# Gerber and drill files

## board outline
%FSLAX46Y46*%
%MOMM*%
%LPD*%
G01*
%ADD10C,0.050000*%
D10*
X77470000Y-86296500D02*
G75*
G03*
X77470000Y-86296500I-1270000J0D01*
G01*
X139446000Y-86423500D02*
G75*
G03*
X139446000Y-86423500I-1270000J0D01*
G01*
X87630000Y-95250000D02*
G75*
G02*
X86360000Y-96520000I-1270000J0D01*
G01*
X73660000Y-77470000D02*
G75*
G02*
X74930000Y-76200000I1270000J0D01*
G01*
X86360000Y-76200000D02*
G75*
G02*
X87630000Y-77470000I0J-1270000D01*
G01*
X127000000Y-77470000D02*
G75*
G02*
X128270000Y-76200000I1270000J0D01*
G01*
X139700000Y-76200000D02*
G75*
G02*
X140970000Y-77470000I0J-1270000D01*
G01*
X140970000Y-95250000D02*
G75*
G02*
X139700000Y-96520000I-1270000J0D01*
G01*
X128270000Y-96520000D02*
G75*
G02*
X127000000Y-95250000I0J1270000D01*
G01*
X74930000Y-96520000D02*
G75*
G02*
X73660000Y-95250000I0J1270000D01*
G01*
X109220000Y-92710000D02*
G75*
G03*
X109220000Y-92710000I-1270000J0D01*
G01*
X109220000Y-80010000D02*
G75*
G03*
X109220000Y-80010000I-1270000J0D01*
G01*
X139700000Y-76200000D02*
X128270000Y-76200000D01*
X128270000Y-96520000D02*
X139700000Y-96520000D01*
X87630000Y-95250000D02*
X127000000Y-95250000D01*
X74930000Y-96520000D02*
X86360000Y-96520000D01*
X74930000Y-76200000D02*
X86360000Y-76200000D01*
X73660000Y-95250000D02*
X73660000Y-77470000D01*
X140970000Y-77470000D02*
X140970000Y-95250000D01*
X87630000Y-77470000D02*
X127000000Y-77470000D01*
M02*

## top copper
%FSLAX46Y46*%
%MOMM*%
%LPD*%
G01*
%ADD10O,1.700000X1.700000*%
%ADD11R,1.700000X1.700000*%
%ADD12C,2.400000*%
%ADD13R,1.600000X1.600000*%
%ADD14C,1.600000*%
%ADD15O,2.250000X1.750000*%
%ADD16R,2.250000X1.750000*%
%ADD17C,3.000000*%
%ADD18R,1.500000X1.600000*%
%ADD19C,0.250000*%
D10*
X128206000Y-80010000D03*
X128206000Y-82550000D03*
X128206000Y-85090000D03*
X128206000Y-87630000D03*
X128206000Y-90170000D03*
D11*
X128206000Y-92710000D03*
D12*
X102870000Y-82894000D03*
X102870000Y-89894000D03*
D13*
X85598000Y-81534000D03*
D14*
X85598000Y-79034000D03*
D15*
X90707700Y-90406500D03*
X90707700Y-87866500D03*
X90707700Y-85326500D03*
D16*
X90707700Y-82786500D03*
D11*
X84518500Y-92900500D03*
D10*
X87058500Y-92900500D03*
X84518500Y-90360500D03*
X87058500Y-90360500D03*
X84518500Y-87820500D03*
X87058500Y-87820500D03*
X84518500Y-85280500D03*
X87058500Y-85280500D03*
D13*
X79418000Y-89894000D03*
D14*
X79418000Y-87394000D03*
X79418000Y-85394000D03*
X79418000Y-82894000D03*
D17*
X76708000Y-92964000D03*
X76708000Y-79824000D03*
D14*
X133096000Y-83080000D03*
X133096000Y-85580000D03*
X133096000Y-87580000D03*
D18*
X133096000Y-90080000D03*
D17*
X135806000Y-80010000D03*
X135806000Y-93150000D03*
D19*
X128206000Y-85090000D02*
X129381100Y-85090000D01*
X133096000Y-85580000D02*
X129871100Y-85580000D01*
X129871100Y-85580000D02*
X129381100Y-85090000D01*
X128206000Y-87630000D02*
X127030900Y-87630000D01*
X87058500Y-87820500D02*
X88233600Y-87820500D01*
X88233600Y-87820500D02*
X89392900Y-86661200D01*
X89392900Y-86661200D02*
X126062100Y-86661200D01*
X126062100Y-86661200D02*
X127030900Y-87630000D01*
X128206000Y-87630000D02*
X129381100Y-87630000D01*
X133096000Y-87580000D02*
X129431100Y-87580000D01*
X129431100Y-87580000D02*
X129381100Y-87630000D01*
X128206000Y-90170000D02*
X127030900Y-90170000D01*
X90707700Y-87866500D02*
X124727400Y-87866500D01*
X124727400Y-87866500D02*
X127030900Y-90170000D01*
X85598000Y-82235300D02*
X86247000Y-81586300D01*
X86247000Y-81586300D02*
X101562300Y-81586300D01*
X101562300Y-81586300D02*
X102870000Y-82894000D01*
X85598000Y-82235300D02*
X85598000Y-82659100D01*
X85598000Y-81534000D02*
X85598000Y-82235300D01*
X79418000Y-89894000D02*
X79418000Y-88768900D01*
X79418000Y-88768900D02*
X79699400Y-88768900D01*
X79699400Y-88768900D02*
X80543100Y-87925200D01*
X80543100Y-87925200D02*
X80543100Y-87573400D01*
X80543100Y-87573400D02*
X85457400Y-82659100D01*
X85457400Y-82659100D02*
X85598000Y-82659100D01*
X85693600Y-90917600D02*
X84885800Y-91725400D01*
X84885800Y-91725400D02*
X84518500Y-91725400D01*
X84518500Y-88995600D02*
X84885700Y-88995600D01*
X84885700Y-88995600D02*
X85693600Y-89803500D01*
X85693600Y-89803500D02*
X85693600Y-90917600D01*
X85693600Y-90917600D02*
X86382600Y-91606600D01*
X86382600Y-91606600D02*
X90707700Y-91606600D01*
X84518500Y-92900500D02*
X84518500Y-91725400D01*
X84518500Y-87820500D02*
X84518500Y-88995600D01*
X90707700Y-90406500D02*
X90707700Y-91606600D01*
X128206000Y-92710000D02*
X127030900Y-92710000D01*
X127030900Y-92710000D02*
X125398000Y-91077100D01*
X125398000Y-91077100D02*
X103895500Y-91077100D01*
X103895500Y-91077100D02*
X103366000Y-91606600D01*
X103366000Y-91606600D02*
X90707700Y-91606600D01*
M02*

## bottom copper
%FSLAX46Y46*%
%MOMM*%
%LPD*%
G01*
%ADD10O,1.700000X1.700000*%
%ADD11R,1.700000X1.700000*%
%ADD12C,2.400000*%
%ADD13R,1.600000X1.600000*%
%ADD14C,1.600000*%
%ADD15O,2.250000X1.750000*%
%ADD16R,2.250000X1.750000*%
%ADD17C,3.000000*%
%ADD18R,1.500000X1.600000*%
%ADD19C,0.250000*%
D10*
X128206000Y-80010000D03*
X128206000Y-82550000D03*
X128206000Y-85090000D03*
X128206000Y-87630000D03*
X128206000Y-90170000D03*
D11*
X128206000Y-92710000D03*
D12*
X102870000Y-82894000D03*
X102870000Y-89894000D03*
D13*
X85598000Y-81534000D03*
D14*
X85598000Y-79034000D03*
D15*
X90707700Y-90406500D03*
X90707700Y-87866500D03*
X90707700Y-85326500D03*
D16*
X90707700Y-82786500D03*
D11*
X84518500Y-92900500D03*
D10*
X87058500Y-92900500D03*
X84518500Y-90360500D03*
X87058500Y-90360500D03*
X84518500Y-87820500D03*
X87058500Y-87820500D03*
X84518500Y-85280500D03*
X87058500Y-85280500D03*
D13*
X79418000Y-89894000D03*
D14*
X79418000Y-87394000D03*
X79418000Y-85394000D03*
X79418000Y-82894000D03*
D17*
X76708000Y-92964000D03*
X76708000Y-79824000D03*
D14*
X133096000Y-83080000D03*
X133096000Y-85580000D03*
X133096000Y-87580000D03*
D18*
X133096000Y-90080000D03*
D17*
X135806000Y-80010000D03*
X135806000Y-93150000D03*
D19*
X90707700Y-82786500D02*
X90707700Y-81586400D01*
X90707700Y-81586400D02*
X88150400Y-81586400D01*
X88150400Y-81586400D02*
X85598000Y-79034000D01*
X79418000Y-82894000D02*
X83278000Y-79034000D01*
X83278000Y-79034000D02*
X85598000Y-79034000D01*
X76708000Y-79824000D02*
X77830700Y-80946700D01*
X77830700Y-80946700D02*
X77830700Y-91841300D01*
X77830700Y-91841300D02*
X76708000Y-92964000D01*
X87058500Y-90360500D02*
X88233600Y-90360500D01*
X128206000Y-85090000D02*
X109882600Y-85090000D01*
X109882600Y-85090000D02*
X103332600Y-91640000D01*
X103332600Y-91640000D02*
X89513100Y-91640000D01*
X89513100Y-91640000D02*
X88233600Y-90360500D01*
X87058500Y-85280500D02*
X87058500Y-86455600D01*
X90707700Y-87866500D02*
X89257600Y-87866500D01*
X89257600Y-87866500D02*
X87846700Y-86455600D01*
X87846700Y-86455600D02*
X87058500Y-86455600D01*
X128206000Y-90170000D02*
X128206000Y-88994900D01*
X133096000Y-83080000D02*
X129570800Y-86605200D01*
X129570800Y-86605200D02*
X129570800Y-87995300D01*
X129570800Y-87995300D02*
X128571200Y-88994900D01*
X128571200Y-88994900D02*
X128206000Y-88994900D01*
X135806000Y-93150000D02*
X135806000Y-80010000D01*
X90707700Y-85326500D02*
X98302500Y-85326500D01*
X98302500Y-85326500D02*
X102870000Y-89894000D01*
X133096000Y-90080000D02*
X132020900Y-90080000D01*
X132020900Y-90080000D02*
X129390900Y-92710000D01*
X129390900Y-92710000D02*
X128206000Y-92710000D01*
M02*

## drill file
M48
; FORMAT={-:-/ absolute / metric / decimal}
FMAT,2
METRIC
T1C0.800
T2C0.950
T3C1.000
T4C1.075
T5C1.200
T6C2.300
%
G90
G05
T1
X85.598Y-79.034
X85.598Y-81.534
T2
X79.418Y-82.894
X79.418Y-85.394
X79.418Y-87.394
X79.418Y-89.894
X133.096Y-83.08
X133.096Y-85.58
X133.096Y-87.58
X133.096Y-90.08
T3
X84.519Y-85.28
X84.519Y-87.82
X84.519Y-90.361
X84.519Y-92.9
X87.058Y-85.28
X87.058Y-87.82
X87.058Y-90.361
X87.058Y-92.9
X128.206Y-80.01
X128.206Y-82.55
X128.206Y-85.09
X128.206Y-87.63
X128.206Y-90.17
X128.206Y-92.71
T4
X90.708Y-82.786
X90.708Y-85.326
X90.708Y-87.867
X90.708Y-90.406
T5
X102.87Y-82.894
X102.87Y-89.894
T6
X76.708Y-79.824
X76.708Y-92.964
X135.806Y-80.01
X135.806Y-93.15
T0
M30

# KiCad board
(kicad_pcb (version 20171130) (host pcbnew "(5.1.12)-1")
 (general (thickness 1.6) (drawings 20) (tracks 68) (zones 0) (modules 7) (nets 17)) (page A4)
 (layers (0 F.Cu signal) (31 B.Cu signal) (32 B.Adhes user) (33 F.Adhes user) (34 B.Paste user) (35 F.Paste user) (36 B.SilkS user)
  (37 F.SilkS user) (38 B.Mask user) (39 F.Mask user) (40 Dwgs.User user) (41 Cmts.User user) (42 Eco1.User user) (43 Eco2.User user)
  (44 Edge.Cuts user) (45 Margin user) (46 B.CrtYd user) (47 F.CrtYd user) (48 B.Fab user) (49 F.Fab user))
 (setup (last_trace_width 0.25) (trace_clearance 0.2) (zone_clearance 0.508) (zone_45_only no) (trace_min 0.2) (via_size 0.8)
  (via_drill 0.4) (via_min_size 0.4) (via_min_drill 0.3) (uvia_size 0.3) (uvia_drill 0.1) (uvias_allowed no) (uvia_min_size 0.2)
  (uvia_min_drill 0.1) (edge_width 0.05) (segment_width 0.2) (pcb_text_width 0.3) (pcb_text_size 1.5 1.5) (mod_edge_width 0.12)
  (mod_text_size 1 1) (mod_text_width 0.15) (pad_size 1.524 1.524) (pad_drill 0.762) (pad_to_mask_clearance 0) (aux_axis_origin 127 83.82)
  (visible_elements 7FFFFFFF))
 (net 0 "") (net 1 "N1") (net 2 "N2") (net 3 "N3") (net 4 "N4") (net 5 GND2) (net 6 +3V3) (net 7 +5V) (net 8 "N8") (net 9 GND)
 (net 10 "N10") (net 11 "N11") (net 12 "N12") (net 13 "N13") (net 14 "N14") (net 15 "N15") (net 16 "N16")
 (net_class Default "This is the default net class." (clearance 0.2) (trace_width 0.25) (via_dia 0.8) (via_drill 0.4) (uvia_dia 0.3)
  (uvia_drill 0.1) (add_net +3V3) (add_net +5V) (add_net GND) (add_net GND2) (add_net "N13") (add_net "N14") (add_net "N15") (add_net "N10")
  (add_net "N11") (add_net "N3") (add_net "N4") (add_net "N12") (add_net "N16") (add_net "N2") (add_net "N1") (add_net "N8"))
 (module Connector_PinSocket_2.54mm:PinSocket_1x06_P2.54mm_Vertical (layer F.Cu) (at 128.206 92.71 180)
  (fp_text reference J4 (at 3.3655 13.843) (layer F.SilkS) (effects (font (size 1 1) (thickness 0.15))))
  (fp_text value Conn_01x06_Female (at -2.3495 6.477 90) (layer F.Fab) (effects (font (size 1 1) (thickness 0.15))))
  (pad 6 thru_hole oval (at 0 12.7 180) (size 1.7 1.7) (drill 1) (layers *.Cu *.Mask) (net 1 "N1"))
  (pad 5 thru_hole oval (at 0 10.16 180) (size 1.7 1.7) (drill 1) (layers *.Cu *.Mask) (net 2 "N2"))
  (pad 4 thru_hole oval (at 0 7.62 180) (size 1.7 1.7) (drill 1) (layers *.Cu *.Mask) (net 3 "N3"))
  (pad 3 thru_hole oval (at 0 5.08 180) (size 1.7 1.7) (drill 1) (layers *.Cu *.Mask) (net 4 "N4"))
  (pad 2 thru_hole oval (at 0 2.54 180) (size 1.7 1.7) (drill 1) (layers *.Cu *.Mask) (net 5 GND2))
  (pad 1 thru_hole rect (at 0 0 180) (size 1.7 1.7) (drill 1) (layers *.Cu *.Mask) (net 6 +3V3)))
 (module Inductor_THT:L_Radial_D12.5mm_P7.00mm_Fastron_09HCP (layer F.Cu) (at 102.87 82.894 270)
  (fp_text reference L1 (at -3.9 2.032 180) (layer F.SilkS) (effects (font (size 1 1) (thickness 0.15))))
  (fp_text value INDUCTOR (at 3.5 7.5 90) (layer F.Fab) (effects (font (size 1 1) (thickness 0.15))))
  (pad 1 thru_hole circle (at 0 0 270) (size 2.4 2.4) (drill 1.2) (layers *.Cu *.Mask) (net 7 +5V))
  (pad 2 thru_hole circle (at 7 0 270) (size 2.4 2.4) (drill 1.2) (layers *.Cu *.Mask) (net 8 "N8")))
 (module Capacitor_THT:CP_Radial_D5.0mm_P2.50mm (layer F.Cu) (at 85.598 81.534 90)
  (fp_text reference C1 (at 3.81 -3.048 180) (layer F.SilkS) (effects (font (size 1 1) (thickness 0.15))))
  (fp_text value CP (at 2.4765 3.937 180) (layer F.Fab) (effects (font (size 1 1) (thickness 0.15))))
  (pad 1 thru_hole rect (at 0 0 90) (size 1.6 1.6) (drill 0.8) (layers *.Cu *.Mask) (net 7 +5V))
  (pad 2 thru_hole circle (at 2.5 0 90) (size 1.6 1.6) (drill 0.8) (layers *.Cu *.Mask) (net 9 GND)))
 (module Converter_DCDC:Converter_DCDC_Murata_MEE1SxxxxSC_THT (layer F.Cu) (at 90.7077 82.7865)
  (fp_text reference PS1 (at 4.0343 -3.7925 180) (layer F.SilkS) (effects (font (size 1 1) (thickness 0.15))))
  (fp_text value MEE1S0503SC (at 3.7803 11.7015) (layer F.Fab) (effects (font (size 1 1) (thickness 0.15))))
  (pad 4 thru_hole oval (at 0 7.62 270) (size 1.75 2.25) (drill 1.075) (layers *.Cu *.Mask) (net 6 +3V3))
  (pad 3 thru_hole oval (at 0 5.08 270) (size 1.75 2.25) (drill 1.075) (layers *.Cu *.Mask) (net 5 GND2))
  (pad 2 thru_hole oval (at 0 2.54 270) (size 1.75 2.25) (drill 1.075) (layers *.Cu *.Mask) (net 8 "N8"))
  (pad 1 thru_hole rect (at 0 0 270) (size 1.75 2.25) (drill 1.075) (layers *.Cu *.Mask) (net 9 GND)))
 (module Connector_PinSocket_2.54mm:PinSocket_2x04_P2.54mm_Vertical (layer F.Cu) (at 84.5185 92.9005 180)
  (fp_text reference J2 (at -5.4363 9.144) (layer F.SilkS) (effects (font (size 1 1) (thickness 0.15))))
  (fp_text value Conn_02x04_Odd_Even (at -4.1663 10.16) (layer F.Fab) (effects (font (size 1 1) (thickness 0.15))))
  (pad 1 thru_hole rect (at 0 0 180) (size 1.7 1.7) (drill 1) (layers *.Cu *.Mask) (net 6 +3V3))
  (pad 2 thru_hole oval (at -2.54 0 180) (size 1.7 1.7) (drill 1) (layers *.Cu *.Mask) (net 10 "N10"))
  (pad 3 thru_hole oval (at 0 2.54 180) (size 1.7 1.7) (drill 1) (layers *.Cu *.Mask) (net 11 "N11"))
  (pad 4 thru_hole oval (at -2.54 2.54 180) (size 1.7 1.7) (drill 1) (layers *.Cu *.Mask) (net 3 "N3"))
  (pad 5 thru_hole oval (at 0 5.08 180) (size 1.7 1.7) (drill 1) (layers *.Cu *.Mask) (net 6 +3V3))
  (pad 6 thru_hole oval (at -2.54 5.08 180) (size 1.7 1.7) (drill 1) (layers *.Cu *.Mask) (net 4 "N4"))
  (pad 7 thru_hole oval (at 0 7.62 180) (size 1.7 1.7) (drill 1) (layers *.Cu *.Mask) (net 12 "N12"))
  (pad 8 thru_hole oval (at -2.54 7.62 180) (size 1.7 1.7) (drill 1) (layers *.Cu *.Mask) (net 5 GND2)))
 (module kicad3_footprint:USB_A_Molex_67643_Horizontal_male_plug (layer F.Cu) (at 79.418 82.894 270)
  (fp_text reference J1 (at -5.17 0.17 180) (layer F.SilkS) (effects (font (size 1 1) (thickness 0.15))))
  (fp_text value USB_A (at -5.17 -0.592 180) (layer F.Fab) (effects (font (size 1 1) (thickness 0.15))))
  (pad 1 thru_hole rect (at 7 0 270) (size 1.6 1.6) (drill 0.95) (layers *.Cu *.Mask) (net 7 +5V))
  (pad 2 thru_hole circle (at 4.5 0 270) (size 1.6 1.6) (drill 0.95) (layers *.Cu *.Mask) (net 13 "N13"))
  (pad 3 thru_hole circle (at 2.5 0 270) (size 1.6 1.6) (drill 0.95) (layers *.Cu *.Mask) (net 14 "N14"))
  (pad 4 thru_hole circle (at 0 0 270) (size 1.6 1.6) (drill 0.95) (layers *.Cu *.Mask) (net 9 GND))
  (pad 5 thru_hole circle (at 10.07 2.71 270) (size 3 3) (drill 2.3) (layers *.Cu *.Mask) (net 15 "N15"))
  (pad 5 thru_hole circle (at -3.07 2.71 270) (size 3 3) (drill 2.3) (layers *.Cu *.Mask) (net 15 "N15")))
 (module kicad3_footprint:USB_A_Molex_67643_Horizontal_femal (layer F.Cu) (at 133.096 90.08 90)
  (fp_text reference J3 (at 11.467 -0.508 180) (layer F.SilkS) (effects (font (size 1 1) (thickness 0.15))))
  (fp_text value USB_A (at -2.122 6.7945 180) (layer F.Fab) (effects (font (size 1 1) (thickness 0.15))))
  (pad 4 thru_hole circle (at 7 0 90) (size 1.6 1.6) (drill 0.95) (layers *.Cu *.Mask) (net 5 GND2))
  (pad 3 thru_hole circle (at 4.5 0 90) (size 1.6 1.6) (drill 0.95) (layers *.Cu *.Mask) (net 3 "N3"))
  (pad 2 thru_hole circle (at 2.5 0 90) (size 1.6 1.6) (drill 0.95) (layers *.Cu *.Mask) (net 4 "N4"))
  (pad 1 thru_hole rect (at 0 0 90) (size 1.6 1.5) (drill 0.95) (layers *.Cu *.Mask) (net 6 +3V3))
  (pad 5 thru_hole circle (at 10.07 2.71 90) (size 3 3) (drill 2.3) (layers *.Cu *.Mask) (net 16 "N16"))
  (pad 5 thru_hole circle (at -3.07 2.71 90) (size 3 3) (drill 2.3) (layers *.Cu *.Mask) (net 16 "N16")))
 (gr_circle (center 76.2 86.2965) (end 76.2 85.0265) (layer Edge.Cuts) (width 0.05))
 (gr_circle (center 138.176 86.4235) (end 138.176 85.1535) (layer Edge.Cuts) (width 0.05))
 (gr_arc (start 86.36 95.25) (end 86.36 96.52) (angle -90) (layer Edge.Cuts) (width 0.05))
 (gr_arc (start 74.93 77.47) (end 74.93 76.2) (angle -90) (layer Edge.Cuts) (width 0.05))
 (gr_arc (start 86.36 77.47) (end 87.63 77.47) (angle -90) (layer Edge.Cuts) (width 0.05))
 (gr_arc (start 128.27 77.47) (end 128.27 76.2) (angle -90) (layer Edge.Cuts) (width 0.05))
 (gr_arc (start 139.7 77.47) (end 140.97 77.47) (angle -90) (layer Edge.Cuts) (width 0.05))
 (gr_arc (start 139.7 95.25) (end 139.7 96.52) (angle -90) (layer Edge.Cuts) (width 0.05))
 (gr_arc (start 128.27 95.25) (end 127 95.25) (angle -90) (layer Edge.Cuts) (width 0.05))
 (gr_arc (start 74.93 95.25) (end 73.66 95.25) (angle -90) (layer Edge.Cuts) (width 0.05))
 (gr_circle (center 107.95 92.71) (end 107.95 93.98) (layer Edge.Cuts) (width 0.05))
 (gr_circle (center 107.95 80.01) (end 107.95 78.74) (layer Edge.Cuts) (width 0.05))
 (gr_line (start 139.7 76.2) (end 128.27 76.2) (layer Edge.Cuts) (width 0.05))
 (gr_line (start 128.27 96.52) (end 139.7 96.52) (layer Edge.Cuts) (width 0.05))
 (gr_line (start 87.63 95.25) (end 127 95.25) (layer Edge.Cuts) (width 0.05))
 (gr_line (start 74.93 96.52) (end 86.36 96.52) (layer Edge.Cuts) (width 0.05))
 (gr_line (start 74.93 76.2) (end 86.36 76.2) (layer Edge.Cuts) (width 0.05))
 (gr_line (start 73.66 95.25) (end 73.66 77.47) (layer Edge.Cuts) (width 0.05))
 (gr_line (start 140.97 77.47) (end 140.97 95.25) (layer Edge.Cuts) (width 0.05))
 (gr_line (start 87.63 77.47) (end 127 77.47) (layer Edge.Cuts) (width 0.05))
 (segment (start 90.7077 82.7865) (end 90.7077 81.5864) (width 0.25) (layer B.Cu) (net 9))
 (segment (start 90.7077 81.5864) (end 88.1504 81.5864) (width 0.25) (layer B.Cu) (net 9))
 (segment (start 88.1504 81.5864) (end 85.598 79.034) (width 0.25) (layer B.Cu) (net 9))
 (segment (start 79.418 82.894) (end 83.278 79.034) (width 0.25) (layer B.Cu) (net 9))
 (segment (start 83.278 79.034) (end 85.598 79.034) (width 0.25) (layer B.Cu) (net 9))
 (segment (start 76.708 79.824) (end 77.8307 80.9467) (width 0.25) (layer B.Cu) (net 15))
 (segment (start 77.8307 80.9467) (end 77.8307 91.8413) (width 0.25) (layer B.Cu) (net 15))
 (segment (start 77.8307 91.8413) (end 76.708 92.964) (width 0.25) (layer B.Cu) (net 15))
 (segment (start 87.0585 90.3605) (end 88.2336 90.3605) (width 0.25) (layer B.Cu) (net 3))
 (segment (start 128.206 85.09) (end 109.8826 85.09) (width 0.25) (layer B.Cu) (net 3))
 (segment (start 109.8826 85.09) (end 103.3326 91.64) (width 0.25) (layer B.Cu) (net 3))
 (segment (start 103.3326 91.64) (end 89.5131 91.64) (width 0.25) (layer B.Cu) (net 3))
 (segment (start 89.5131 91.64) (end 88.2336 90.3605) (width 0.25) (layer B.Cu) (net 3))
 (segment (start 128.206 85.09) (end 129.3811 85.09) (width 0.25) (layer F.Cu) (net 3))
 (segment (start 133.096 85.58) (end 129.8711 85.58) (width 0.25) (layer F.Cu) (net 3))
 (segment (start 129.8711 85.58) (end 129.3811 85.09) (width 0.25) (layer F.Cu) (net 3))
 (segment (start 128.206 87.63) (end 127.0309 87.63) (width 0.25) (layer F.Cu) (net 4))
 (segment (start 87.0585 87.8205) (end 88.2336 87.8205) (width 0.25) (layer F.Cu) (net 4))
 (segment (start 88.2336 87.8205) (end 89.3929 86.6612) (width 0.25) (layer F.Cu) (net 4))
 (segment (start 89.3929 86.6612) (end 126.0621 86.6612) (width 0.25) (layer F.Cu) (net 4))
 (segment (start 126.0621 86.6612) (end 127.0309 87.63) (width 0.25) (layer F.Cu) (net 4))
 (segment (start 128.206 87.63) (end 129.3811 87.63) (width 0.25) (layer F.Cu) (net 4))
 (segment (start 133.096 87.58) (end 129.4311 87.58) (width 0.25) (layer F.Cu) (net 4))
 (segment (start 129.4311 87.58) (end 129.3811 87.63) (width 0.25) (layer F.Cu) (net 4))
 (segment (start 87.0585 85.2805) (end 87.0585 86.4556) (width 0.25) (layer B.Cu) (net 5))
 (segment (start 90.7077 87.8665) (end 89.2576 87.8665) (width 0.25) (layer B.Cu) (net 5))
 (segment (start 89.2576 87.8665) (end 87.8467 86.4556) (width 0.25) (layer B.Cu) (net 5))
 (segment (start 87.8467 86.4556) (end 87.0585 86.4556) (width 0.25) (layer B.Cu) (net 5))
 (segment (start 128.206 90.17) (end 127.0309 90.17) (width 0.25) (layer F.Cu) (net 5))
 (segment (start 90.7077 87.8665) (end 124.7274 87.8665) (width 0.25) (layer F.Cu) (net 5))
 (segment (start 124.7274 87.8665) (end 127.0309 90.17) (width 0.25) (layer F.Cu) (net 5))
 (segment (start 128.206 90.17) (end 128.206 88.9949) (width 0.25) (layer B.Cu) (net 5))
 (segment (start 133.096 83.08) (end 129.5708 86.6052) (width 0.25) (layer B.Cu) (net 5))
 (segment (start 129.5708 86.6052) (end 129.5708 87.9953) (width 0.25) (layer B.Cu) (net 5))
 (segment (start 129.5708 87.9953) (end 128.5712 88.9949) (width 0.25) (layer B.Cu) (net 5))
 (segment (start 128.5712 88.9949) (end 128.206 88.9949) (width 0.25) (layer B.Cu) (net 5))
 (segment (start 135.806 93.15) (end 135.806 80.01) (width 0.25) (layer B.Cu) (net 16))
 (segment (start 90.7077 85.3265) (end 98.3025 85.3265) (width 0.25) (layer B.Cu) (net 8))
 (segment (start 98.3025 85.3265) (end 102.87 89.894) (width 0.25) (layer B.Cu) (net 8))
 (segment (start 85.598 82.2353) (end 86.247 81.5863) (width 0.25) (layer F.Cu) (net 7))
 (segment (start 86.247 81.5863) (end 101.5623 81.5863) (width 0.25) (layer F.Cu) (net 7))
 (segment (start 101.5623 81.5863) (end 102.87 82.894) (width 0.25) (layer F.Cu) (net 7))
 (segment (start 85.598 82.2353) (end 85.598 82.6591) (width 0.25) (layer F.Cu) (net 7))
 (segment (start 85.598 81.534) (end 85.598 82.2353) (width 0.25) (layer F.Cu) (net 7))
 (segment (start 79.418 89.894) (end 79.418 88.7689) (width 0.25) (layer F.Cu) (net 7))
 (segment (start 79.418 88.7689) (end 79.6994 88.7689) (width 0.25) (layer F.Cu) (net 7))
 (segment (start 79.6994 88.7689) (end 80.5431 87.9252) (width 0.25) (layer F.Cu) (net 7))
 (segment (start 80.5431 87.9252) (end 80.5431 87.5734) (width 0.25) (layer F.Cu) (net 7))
 (segment (start 80.5431 87.5734) (end 85.4574 82.6591) (width 0.25) (layer F.Cu) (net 7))
 (segment (start 85.4574 82.6591) (end 85.598 82.6591) (width 0.25) (layer F.Cu) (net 7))
 (segment (start 85.6936 90.9176) (end 84.8858 91.7254) (width 0.25) (layer F.Cu) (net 6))
 (segment (start 84.8858 91.7254) (end 84.5185 91.7254) (width 0.25) (layer F.Cu) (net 6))
 (segment (start 84.5185 88.9956) (end 84.8857 88.9956) (width 0.25) (layer F.Cu) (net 6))
 (segment (start 84.8857 88.9956) (end 85.6936 89.8035) (width 0.25) (layer F.Cu) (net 6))
 (segment (start 85.6936 89.8035) (end 85.6936 90.9176) (width 0.25) (layer F.Cu) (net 6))
 (segment (start 85.6936 90.9176) (end 86.3826 91.6066) (width 0.25) (layer F.Cu) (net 6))
 (segment (start 86.3826 91.6066) (end 90.7077 91.6066) (width 0.25) (layer F.Cu) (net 6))
 (segment (start 84.5185 92.9005) (end 84.5185 91.7254) (width 0.25) (layer F.Cu) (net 6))
 (segment (start 84.5185 87.8205) (end 84.5185 88.9956) (width 0.25) (layer F.Cu) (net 6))
 (segment (start 90.7077 90.4065) (end 90.7077 91.6066) (width 0.25) (layer F.Cu) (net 6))
 (segment (start 128.206 92.71) (end 127.0309 92.71) (width 0.25) (layer F.Cu) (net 6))
 (segment (start 127.0309 92.71) (end 125.398 91.0771) (width 0.25) (layer F.Cu) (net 6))
 (segment (start 125.398 91.0771) (end 103.8955 91.0771) (width 0.25) (layer F.Cu) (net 6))
 (segment (start 103.8955 91.0771) (end 103.366 91.6066) (width 0.25) (layer F.Cu) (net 6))
 (segment (start 103.366 91.6066) (end 90.7077 91.6066) (width 0.25) (layer F.Cu) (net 6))
 (segment (start 133.096 90.08) (end 132.0209 90.08) (width 0.25) (layer B.Cu) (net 6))
 (segment (start 132.0209 90.08) (end 129.3909 92.71) (width 0.25) (layer B.Cu) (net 6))
 (segment (start 129.3909 92.71) (end 128.206 92.71) (width 0.25) (layer B.Cu) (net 6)))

